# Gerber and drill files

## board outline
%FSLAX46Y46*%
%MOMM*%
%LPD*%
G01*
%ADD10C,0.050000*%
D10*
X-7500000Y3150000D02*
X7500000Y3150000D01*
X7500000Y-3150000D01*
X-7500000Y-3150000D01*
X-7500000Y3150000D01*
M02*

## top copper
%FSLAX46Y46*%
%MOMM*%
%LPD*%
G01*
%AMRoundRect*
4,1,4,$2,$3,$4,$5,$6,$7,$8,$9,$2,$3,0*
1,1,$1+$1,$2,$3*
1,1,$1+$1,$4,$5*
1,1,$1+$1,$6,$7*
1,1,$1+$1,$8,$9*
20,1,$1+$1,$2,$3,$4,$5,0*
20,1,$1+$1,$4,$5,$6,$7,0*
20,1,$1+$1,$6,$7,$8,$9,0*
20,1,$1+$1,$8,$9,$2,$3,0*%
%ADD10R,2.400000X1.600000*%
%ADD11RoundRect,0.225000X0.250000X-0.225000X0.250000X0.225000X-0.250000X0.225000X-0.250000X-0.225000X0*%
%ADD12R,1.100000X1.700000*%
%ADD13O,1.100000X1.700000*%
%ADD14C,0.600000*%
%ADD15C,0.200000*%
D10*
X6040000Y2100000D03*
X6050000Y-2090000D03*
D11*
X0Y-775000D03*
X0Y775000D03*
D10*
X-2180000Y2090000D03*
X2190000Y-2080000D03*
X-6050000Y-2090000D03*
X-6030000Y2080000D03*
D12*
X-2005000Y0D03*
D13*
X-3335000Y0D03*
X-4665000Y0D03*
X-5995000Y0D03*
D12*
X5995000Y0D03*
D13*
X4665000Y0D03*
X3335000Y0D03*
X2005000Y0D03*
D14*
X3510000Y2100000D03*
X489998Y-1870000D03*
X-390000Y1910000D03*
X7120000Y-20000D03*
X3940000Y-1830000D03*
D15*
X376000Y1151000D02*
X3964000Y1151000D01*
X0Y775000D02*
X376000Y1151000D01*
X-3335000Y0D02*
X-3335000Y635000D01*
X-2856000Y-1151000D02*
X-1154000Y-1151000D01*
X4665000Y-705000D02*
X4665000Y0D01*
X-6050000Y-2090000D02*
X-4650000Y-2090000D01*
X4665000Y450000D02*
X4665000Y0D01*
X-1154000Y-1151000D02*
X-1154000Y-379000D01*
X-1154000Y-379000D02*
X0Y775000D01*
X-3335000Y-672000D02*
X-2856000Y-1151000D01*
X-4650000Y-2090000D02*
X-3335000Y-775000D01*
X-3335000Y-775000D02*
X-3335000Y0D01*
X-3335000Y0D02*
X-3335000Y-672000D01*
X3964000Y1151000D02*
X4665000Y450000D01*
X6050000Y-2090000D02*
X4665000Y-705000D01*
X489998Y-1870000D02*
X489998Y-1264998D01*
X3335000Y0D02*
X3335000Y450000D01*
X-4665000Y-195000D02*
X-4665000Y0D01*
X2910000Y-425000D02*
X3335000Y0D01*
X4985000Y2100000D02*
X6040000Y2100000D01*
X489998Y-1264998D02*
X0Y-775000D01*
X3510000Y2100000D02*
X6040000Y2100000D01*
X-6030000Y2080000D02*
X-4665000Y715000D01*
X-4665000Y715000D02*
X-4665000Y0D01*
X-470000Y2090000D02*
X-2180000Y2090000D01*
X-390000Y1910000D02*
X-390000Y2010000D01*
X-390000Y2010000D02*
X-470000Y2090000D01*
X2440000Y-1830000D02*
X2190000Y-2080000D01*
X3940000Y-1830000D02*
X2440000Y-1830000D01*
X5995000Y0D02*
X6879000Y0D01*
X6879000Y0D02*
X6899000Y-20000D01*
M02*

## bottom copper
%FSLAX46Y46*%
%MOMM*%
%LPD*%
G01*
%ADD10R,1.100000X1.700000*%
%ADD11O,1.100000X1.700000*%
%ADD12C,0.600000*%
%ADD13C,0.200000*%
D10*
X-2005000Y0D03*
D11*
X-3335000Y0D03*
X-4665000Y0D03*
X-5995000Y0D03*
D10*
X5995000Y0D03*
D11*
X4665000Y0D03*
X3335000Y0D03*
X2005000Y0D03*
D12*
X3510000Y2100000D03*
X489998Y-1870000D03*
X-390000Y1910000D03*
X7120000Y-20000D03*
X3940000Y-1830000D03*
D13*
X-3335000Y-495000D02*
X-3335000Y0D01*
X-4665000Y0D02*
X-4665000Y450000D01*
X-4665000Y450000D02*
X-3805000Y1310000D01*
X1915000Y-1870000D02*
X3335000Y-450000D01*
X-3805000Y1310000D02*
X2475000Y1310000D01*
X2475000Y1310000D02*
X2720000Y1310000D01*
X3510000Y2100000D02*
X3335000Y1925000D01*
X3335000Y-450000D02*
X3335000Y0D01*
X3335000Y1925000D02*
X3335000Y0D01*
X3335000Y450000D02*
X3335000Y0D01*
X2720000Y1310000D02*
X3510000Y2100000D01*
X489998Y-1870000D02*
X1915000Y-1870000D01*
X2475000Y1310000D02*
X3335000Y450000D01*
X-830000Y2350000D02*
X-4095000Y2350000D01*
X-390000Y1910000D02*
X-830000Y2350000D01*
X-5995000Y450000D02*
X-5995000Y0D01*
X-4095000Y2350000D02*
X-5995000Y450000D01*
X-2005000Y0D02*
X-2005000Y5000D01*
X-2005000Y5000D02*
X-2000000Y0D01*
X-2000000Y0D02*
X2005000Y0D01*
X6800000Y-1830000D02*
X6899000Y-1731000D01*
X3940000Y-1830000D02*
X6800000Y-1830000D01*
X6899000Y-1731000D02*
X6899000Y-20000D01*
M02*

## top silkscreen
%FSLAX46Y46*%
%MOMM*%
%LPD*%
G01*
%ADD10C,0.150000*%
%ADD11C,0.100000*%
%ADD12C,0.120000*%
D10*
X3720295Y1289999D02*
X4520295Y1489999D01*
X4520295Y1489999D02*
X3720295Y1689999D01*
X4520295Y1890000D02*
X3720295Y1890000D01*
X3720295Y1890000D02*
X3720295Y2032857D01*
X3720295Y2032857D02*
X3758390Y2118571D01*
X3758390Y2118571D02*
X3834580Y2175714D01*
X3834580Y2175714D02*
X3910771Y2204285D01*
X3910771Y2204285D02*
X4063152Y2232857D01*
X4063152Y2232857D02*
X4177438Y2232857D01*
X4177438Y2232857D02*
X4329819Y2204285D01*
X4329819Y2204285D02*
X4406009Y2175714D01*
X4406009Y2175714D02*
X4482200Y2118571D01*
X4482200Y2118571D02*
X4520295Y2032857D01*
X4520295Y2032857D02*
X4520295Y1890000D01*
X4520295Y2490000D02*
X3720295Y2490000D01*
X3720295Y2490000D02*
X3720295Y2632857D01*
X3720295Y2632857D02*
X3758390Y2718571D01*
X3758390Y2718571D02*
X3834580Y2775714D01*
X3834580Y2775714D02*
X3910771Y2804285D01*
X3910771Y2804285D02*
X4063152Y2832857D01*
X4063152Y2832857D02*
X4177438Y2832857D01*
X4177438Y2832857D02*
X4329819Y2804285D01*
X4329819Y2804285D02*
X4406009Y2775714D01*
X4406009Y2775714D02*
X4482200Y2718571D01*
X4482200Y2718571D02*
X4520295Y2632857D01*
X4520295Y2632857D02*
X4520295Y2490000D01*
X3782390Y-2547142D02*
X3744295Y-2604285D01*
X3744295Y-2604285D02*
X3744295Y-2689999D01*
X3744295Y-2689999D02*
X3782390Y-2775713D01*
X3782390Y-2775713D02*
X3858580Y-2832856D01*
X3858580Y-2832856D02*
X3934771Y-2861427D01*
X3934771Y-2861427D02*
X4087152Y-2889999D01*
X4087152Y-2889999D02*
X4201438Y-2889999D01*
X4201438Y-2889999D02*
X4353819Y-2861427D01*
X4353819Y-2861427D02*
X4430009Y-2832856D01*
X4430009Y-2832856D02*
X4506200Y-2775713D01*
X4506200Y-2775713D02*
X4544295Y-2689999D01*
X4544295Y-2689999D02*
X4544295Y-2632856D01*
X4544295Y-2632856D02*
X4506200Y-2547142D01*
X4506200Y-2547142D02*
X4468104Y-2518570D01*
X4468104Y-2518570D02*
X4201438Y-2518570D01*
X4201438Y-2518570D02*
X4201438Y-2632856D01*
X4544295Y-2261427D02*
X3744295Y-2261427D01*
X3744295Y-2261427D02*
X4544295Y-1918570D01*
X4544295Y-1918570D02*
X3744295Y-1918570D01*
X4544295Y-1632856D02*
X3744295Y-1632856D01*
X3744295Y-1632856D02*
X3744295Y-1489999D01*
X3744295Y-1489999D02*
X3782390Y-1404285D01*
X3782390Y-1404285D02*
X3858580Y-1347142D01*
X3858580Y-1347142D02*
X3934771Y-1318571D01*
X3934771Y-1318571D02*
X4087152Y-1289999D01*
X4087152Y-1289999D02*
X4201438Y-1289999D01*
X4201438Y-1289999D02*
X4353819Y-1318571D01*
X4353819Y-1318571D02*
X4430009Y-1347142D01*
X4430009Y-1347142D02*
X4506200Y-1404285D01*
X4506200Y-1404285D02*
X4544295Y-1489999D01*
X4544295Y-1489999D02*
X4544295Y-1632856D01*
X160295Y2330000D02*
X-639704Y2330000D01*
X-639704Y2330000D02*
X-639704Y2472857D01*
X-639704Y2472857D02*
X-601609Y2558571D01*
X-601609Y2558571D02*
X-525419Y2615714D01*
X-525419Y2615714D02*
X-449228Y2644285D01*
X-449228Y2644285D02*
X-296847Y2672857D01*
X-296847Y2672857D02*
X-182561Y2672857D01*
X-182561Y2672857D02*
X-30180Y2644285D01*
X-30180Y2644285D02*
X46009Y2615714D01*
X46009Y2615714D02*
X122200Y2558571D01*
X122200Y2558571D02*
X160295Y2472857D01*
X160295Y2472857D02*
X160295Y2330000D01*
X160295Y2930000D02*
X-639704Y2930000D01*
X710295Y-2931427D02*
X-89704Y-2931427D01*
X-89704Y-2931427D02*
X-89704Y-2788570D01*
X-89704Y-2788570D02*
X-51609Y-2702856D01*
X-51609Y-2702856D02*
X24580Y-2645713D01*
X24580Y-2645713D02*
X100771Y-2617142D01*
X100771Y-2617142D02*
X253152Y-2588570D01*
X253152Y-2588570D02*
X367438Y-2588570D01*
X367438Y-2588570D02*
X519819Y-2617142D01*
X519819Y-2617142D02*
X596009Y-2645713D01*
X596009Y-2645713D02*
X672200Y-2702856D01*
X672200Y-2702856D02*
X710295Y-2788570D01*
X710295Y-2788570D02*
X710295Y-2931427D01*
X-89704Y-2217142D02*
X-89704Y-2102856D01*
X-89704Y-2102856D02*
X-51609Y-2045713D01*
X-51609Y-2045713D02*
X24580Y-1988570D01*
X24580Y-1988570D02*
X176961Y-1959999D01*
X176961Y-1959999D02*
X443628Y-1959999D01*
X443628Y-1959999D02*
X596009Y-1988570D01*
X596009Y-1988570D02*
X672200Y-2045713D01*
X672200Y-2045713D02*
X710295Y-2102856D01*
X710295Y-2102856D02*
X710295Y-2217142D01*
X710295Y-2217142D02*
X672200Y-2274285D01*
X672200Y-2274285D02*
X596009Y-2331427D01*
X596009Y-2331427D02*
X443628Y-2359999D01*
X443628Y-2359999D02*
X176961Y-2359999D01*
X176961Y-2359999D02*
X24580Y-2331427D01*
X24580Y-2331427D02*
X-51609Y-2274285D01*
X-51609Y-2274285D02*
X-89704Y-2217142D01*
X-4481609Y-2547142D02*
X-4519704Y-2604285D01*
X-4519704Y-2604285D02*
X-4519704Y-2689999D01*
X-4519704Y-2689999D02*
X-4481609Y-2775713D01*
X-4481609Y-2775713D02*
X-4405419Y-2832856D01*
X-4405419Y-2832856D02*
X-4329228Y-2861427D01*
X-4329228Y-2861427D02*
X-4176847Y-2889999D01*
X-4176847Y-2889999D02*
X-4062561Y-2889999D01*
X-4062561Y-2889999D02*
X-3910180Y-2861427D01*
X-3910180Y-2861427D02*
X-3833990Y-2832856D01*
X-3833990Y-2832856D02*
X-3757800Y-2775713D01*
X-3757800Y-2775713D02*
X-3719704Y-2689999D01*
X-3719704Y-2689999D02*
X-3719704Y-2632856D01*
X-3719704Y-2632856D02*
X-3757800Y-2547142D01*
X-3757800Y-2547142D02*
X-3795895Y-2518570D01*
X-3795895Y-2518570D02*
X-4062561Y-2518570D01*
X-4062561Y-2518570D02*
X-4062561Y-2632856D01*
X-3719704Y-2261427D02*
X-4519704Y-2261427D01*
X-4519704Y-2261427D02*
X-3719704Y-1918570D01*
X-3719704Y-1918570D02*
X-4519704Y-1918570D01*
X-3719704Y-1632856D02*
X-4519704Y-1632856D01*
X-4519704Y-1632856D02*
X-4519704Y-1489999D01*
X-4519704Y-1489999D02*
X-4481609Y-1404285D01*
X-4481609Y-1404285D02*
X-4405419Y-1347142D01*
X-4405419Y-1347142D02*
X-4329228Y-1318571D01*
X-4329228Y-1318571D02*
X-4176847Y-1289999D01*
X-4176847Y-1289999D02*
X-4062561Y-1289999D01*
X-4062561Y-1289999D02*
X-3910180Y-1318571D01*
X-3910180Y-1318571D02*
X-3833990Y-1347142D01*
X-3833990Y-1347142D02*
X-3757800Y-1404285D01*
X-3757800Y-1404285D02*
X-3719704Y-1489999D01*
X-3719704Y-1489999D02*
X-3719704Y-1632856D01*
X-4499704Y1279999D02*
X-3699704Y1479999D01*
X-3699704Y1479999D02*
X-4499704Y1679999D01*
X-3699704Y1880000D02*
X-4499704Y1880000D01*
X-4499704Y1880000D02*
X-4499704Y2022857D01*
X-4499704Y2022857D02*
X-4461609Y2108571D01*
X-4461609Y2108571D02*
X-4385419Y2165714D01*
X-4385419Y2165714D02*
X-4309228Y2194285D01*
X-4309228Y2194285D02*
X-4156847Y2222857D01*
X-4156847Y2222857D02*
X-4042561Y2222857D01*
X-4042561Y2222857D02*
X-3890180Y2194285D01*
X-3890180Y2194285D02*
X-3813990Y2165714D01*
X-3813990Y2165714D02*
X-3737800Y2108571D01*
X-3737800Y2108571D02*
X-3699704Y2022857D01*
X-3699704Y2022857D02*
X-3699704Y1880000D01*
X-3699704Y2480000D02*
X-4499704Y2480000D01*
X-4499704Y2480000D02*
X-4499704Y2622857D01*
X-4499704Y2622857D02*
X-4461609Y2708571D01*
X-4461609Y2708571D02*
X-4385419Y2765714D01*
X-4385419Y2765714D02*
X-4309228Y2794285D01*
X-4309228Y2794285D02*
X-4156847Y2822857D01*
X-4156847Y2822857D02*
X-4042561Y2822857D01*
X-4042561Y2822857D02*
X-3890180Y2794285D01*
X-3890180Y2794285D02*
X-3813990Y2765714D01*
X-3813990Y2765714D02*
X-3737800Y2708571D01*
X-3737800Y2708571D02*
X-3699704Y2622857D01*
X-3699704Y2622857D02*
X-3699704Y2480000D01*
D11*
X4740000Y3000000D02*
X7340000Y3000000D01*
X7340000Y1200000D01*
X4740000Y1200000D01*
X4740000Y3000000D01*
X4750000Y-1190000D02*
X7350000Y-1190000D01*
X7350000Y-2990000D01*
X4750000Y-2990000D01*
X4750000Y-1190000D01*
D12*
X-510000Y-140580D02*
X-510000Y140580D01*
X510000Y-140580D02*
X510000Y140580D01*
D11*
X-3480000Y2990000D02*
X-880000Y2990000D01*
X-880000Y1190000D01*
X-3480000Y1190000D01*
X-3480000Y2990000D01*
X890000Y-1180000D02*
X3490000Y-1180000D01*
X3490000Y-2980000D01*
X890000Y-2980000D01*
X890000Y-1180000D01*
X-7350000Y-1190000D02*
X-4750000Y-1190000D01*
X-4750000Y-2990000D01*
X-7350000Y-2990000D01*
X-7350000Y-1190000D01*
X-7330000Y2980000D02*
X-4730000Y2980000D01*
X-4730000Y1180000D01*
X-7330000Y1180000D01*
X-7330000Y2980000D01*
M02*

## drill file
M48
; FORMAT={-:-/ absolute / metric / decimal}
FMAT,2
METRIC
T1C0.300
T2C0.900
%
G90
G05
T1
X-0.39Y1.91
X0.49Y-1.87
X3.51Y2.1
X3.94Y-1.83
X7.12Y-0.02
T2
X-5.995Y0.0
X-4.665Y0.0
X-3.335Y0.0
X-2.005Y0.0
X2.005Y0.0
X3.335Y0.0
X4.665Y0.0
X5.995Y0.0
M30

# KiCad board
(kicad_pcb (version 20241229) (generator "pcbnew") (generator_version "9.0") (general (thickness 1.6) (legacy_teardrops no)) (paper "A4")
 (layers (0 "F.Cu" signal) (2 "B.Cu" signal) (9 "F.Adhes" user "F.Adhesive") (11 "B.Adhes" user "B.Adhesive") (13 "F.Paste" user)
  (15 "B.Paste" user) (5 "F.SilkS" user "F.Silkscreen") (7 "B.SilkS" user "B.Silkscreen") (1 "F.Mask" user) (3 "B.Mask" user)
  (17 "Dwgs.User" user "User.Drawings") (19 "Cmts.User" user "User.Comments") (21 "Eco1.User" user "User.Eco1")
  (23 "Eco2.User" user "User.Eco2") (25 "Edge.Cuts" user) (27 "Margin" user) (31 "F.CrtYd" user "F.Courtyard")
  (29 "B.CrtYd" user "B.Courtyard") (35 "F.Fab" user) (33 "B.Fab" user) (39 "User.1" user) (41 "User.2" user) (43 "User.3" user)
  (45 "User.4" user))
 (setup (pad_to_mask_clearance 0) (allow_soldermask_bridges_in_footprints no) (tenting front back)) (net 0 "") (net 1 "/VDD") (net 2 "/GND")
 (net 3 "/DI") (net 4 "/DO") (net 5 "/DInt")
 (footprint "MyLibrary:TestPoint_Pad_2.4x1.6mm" (layer "F.Cu") (at 6.04 -2.1)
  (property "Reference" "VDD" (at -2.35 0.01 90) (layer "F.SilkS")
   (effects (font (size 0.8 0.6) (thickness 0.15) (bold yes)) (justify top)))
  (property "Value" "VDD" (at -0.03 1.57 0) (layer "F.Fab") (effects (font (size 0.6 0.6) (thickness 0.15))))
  (fp_rect (start -1.3 -0.9) (end 1.3 0.9) (stroke (width 0.1) (type solid)) (fill no) (layer "F.SilkS"))
  (pad "1" smd rect (at 0 0) (size 2.4 1.6) (layers "F.Cu" "F.Mask") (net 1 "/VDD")))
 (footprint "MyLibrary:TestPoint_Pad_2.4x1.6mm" (layer "F.Cu") (at 6.05 2.09)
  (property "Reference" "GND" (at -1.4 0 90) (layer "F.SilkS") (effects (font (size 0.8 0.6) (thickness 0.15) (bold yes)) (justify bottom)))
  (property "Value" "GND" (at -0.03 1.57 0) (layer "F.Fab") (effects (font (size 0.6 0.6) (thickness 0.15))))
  (fp_rect (start -1.3 -0.9) (end 1.3 0.9) (stroke (width 0.1) (type solid)) (fill no) (layer "F.SilkS"))
  (pad "1" smd rect (at 0 0) (size 2.4 1.6) (layers "F.Cu" "F.Mask") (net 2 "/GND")))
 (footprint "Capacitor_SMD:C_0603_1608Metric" (layer "F.Cu") (at 0 0 90)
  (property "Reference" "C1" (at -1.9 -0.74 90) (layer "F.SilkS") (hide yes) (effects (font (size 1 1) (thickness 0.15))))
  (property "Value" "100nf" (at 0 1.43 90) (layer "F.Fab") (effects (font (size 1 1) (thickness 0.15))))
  (fp_line (start -0.14058 -0.51) (end 0.14058 -0.51) (stroke (width 0.12) (type solid)) (layer "F.SilkS"))
  (fp_line (start -0.14058 0.51) (end 0.14058 0.51) (stroke (width 0.12) (type solid)) (layer "F.SilkS"))
  (pad "1" smd roundrect (at -0.775 0 90) (size 0.9 0.95) (layers "F.Cu" "F.Mask" "F.Paste") (roundrect_rratio 0.25) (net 1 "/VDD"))
  (pad "2" smd roundrect (at 0.775 0 90) (size 0.9 0.95) (layers "F.Cu" "F.Mask" "F.Paste") (roundrect_rratio 0.25) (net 2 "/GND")))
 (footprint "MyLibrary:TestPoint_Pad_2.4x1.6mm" (layer "F.Cu") (at -2.18 -2.09)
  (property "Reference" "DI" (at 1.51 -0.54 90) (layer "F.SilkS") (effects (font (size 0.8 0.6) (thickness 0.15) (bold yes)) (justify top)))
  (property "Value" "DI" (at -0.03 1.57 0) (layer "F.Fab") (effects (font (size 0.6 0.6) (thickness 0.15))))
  (fp_rect (start -1.3 -0.9) (end 1.3 0.9) (stroke (width 0.1) (type solid)) (fill no) (layer "F.SilkS"))
  (pad "1" smd rect (at 0 0) (size 2.4 1.6) (layers "F.Cu" "F.Mask") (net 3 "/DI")))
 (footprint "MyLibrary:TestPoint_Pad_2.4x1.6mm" (layer "F.Cu") (at 2.19 2.08)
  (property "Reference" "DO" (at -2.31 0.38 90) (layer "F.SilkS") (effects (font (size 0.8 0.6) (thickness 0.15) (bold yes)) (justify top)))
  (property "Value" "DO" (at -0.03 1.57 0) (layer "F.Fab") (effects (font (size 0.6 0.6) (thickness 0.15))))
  (fp_rect (start -1.3 -0.9) (end 1.3 0.9) (stroke (width 0.1) (type solid)) (fill no) (layer "F.SilkS"))
  (pad "1" smd rect (at 0 0) (size 2.4 1.6) (layers "F.Cu" "F.Mask") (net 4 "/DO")))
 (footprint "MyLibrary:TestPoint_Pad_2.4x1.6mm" (layer "F.Cu") (at -6.05 2.09)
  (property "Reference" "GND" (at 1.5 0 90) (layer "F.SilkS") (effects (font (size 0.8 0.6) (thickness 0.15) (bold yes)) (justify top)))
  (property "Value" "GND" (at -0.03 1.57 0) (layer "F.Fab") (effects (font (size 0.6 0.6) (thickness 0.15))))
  (fp_rect (start -1.3 -0.9) (end 1.3 0.9) (stroke (width 0.1) (type solid)) (fill no) (layer "F.SilkS"))
  (pad "1" smd rect (at 0 0) (size 2.4 1.6) (layers "F.Cu" "F.Mask") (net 2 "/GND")))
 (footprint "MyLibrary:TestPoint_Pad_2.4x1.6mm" (layer "F.Cu") (at -6.03 -2.08)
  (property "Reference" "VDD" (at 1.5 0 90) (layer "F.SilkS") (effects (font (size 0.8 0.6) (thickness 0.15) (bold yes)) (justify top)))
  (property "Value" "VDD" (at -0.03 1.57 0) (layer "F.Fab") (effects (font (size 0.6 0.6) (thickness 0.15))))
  (fp_rect (start -1.3 -0.9) (end 1.3 0.9) (stroke (width 0.1) (type solid)) (fill no) (layer "F.SilkS"))
  (pad "1" smd rect (at 0 0) (size 2.4 1.6) (layers "F.Cu" "F.Mask") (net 1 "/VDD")))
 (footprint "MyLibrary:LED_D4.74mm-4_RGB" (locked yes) (layer "B.Cu") (at -4 0 180)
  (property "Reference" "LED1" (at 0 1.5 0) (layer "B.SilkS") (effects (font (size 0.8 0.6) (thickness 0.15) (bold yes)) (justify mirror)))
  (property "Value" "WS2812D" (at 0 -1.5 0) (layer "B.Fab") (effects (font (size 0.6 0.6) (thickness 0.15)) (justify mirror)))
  (pad "1" thru_hole rect (at -1.995 0 180) (size 1.1 1.7) (drill 0.9) (layers "*.Cu" "*.Mask") (remove_unused_layers no) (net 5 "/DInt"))
  (pad "2" thru_hole oval (at -0.665 0 180) (size 1.1 1.7) (drill 0.9) (layers "*.Cu" "*.Mask") (remove_unused_layers no) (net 2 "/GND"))
  (pad "3" thru_hole oval (at 0.665 0 180) (size 1.1 1.7) (drill 0.9) (layers "*.Cu" "*.Mask") (remove_unused_layers no) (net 1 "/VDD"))
  (pad "4" thru_hole oval (at 1.995 0 180) (size 1.1 1.7) (drill 0.9) (layers "*.Cu" "*.Mask") (remove_unused_layers no) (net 3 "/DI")))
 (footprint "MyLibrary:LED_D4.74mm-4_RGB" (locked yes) (layer "B.Cu") (at 4 0 180)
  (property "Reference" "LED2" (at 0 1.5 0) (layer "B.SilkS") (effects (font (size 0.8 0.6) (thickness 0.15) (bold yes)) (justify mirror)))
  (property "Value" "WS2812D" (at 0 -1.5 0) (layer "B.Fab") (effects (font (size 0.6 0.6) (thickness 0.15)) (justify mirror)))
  (pad "1" thru_hole rect (at -1.995 0 180) (size 1.1 1.7) (drill 0.9) (layers "*.Cu" "*.Mask") (remove_unused_layers no) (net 4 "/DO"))
  (pad "2" thru_hole oval (at -0.665 0 180) (size 1.1 1.7) (drill 0.9) (layers "*.Cu" "*.Mask") (remove_unused_layers no) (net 2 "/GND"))
  (pad "3" thru_hole oval (at 0.665 0 180) (size 1.1 1.7) (drill 0.9) (layers "*.Cu" "*.Mask") (remove_unused_layers no) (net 1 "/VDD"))
  (pad "4" thru_hole oval (at 1.995 0 180) (size 1.1 1.7) (drill 0.9) (layers "*.Cu" "*.Mask") (remove_unused_layers no) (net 5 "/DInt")))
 (gr_rect (start -7.5 -3.15) (end 7.5 3.15) (stroke (width 0.05) (type solid)) (fill no) (locked yes) (layer "Edge.Cuts"))
 (segment (start 0.376 -1.151) (end 3.964 -1.151) (width 0.2) (layer "F.Cu") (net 2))
 (segment (start 0 -0.775) (end 0.376 -1.151) (width 0.2) (layer "F.Cu") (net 2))
 (segment (start -3.335 0) (end -3.335 -0.635) (width 0.2) (layer "F.Cu") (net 2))
 (segment (start -2.856 1.151) (end -1.154 1.151) (width 0.2) (layer "F.Cu") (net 2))
 (segment (start 4.665 0.705) (end 4.665 0) (width 0.2) (layer "F.Cu") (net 2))
 (segment (start -6.05 2.09) (end -4.65 2.09) (width 0.2) (layer "F.Cu") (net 2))
 (segment (start 4.665 -0.45) (end 4.665 0) (width 0.2) (layer "F.Cu") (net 2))
 (segment (start -1.154 1.151) (end -1.154 0.379) (width 0.2) (layer "F.Cu") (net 2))
 (segment (start -1.154 0.379) (end 0 -0.775) (width 0.2) (layer "F.Cu") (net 2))
 (segment (start -3.335 0.672) (end -2.856 1.151) (width 0.2) (layer "F.Cu") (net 2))
 (segment (start -4.65 2.09) (end -3.335 0.775) (width 0.2) (layer "F.Cu") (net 2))
 (segment (start -3.335 0.775) (end -3.335 0) (width 0.2) (layer "F.Cu") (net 2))
 (segment (start -3.335 0) (end -3.335 0.672) (width 0.2) (layer "F.Cu") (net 2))
 (segment (start 3.964 -1.151) (end 4.665 -0.45) (width 0.2) (layer "F.Cu") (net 2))
 (segment (start 6.05 2.09) (end 4.665 0.705) (width 0.2) (layer "F.Cu") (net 2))
 (segment (start -3.335 0.495) (end -3.335 0) (width 0.2) (layer "B.Cu") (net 2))
 (segment (start 0.489998 1.87) (end 0.489998 1.264998) (width 0.2) (layer "F.Cu") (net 1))
 (segment (start 3.335 0) (end 3.335 -0.45) (width 0.2) (layer "F.Cu") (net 1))
 (segment (start -4.665 0.195) (end -4.665 0) (width 0.2) (layer "F.Cu") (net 1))
 (segment (start 2.91 0.425) (end 3.335 0) (width 0.2) (layer "F.Cu") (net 1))
 (segment (start 4.985 -2.1) (end 6.04 -2.1) (width 0.2) (layer "F.Cu") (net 1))
 (segment (start 0.489998 1.264998) (end 0 0.775) (width 0.2) (layer "F.Cu") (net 1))
 (segment (start 3.51 -2.1) (end 6.04 -2.1) (width 0.2) (layer "F.Cu") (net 1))
 (segment (start -6.03 -2.08) (end -4.665 -0.715) (width 0.2) (layer "F.Cu") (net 1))
 (segment (start -4.665 -0.715) (end -4.665 0) (width 0.2) (layer "F.Cu") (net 1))
 (via (at 3.51 -2.1) (size 0.6) (drill 0.3) (layers "F.Cu" "B.Cu") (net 1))
 (via (at 0.489998 1.87) (size 0.6) (drill 0.3) (layers "F.Cu" "B.Cu") (free yes) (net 1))
 (segment (start -4.665 0) (end -4.665 -0.45) (width 0.2) (layer "B.Cu") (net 1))
 (segment (start -4.665 -0.45) (end -3.805 -1.31) (width 0.2) (layer "B.Cu") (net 1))
 (segment (start 1.915 1.87) (end 3.335 0.45) (width 0.2) (layer "B.Cu") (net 1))
 (segment (start -3.805 -1.31) (end 2.475 -1.31) (width 0.2) (layer "B.Cu") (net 1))
 (segment (start 2.475 -1.31) (end 2.72 -1.31) (width 0.2) (layer "B.Cu") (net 1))
 (segment (start 3.51 -2.1) (end 3.335 -1.925) (width 0.2) (layer "B.Cu") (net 1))
 (segment (start 3.335 0.45) (end 3.335 0) (width 0.2) (layer "B.Cu") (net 1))
 (segment (start 3.335 -1.925) (end 3.335 0) (width 0.2) (layer "B.Cu") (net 1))
 (segment (start 3.335 -0.45) (end 3.335 0) (width 0.2) (layer "B.Cu") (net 1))
 (segment (start 2.72 -1.31) (end 3.51 -2.1) (width 0.2) (layer "B.Cu") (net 1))
 (segment (start 0.489998 1.87) (end 1.915 1.87) (width 0.2) (layer "B.Cu") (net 1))
 (segment (start 2.475 -1.31) (end 3.335 -0.45) (width 0.2) (layer "B.Cu") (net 1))
 (segment (start -0.47 -2.09) (end -2.18 -2.09) (width 0.2) (layer "F.Cu") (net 3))
 (segment (start -0.39 -1.91) (end -0.39 -2.01) (width 0.2) (layer "F.Cu") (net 3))
 (segment (start -0.39 -2.01) (end -0.47 -2.09) (width 0.2) (layer "F.Cu") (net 3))
 (via (at -0.39 -1.91) (size 0.6) (drill 0.3) (layers "F.Cu" "B.Cu") (free yes) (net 3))
 (segment (start -0.83 -2.35) (end -4.095 -2.35) (width 0.2) (layer "B.Cu") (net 3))
 (segment (start -0.39 -1.91) (end -0.83 -2.35) (width 0.2) (layer "B.Cu") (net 3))
 (segment (start -5.995 -0.45) (end -5.995 0) (width 0.2) (layer "B.Cu") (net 3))
 (segment (start -4.095 -2.35) (end -5.995 -0.45) (width 0.2) (layer "B.Cu") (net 3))
 (segment (start -2.005 0) (end -2.005 -0.005) (width 0.2) (layer "B.Cu") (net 5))
 (segment (start -2.005 -0.005) (end -2 0) (width 0.2) (layer "B.Cu") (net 5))
 (segment (start -2 0) (end 2.005 0) (width 0.2) (layer "B.Cu") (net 5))
 (segment (start 2.44 1.83) (end 2.19 2.08) (width 0.2) (layer "F.Cu") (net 4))
 (segment (start 3.94 1.83) (end 2.44 1.83) (width 0.2) (layer "F.Cu") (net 4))
 (segment (start 5.995 0) (end 6.879 0) (width 0.2) (layer "F.Cu") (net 4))
 (segment (start 6.879 0) (end 6.899 0.02) (width 0.2) (layer "F.Cu") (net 4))
 (via (at 7.12 0.02) (size 0.6) (drill 0.3) (layers "F.Cu" "B.Cu") (free yes) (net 4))
 (via (at 3.94 1.83) (size 0.6) (drill 0.3) (layers "F.Cu" "B.Cu") (free yes) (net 4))
 (segment (start 6.8 1.83) (end 6.899 1.731) (width 0.2) (layer "B.Cu") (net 4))
 (segment (start 3.94 1.83) (end 6.8 1.83) (width 0.2) (layer "B.Cu") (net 4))
 (segment (start 6.899 1.731) (end 6.899 0.02) (width 0.2) (layer "B.Cu") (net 4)))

